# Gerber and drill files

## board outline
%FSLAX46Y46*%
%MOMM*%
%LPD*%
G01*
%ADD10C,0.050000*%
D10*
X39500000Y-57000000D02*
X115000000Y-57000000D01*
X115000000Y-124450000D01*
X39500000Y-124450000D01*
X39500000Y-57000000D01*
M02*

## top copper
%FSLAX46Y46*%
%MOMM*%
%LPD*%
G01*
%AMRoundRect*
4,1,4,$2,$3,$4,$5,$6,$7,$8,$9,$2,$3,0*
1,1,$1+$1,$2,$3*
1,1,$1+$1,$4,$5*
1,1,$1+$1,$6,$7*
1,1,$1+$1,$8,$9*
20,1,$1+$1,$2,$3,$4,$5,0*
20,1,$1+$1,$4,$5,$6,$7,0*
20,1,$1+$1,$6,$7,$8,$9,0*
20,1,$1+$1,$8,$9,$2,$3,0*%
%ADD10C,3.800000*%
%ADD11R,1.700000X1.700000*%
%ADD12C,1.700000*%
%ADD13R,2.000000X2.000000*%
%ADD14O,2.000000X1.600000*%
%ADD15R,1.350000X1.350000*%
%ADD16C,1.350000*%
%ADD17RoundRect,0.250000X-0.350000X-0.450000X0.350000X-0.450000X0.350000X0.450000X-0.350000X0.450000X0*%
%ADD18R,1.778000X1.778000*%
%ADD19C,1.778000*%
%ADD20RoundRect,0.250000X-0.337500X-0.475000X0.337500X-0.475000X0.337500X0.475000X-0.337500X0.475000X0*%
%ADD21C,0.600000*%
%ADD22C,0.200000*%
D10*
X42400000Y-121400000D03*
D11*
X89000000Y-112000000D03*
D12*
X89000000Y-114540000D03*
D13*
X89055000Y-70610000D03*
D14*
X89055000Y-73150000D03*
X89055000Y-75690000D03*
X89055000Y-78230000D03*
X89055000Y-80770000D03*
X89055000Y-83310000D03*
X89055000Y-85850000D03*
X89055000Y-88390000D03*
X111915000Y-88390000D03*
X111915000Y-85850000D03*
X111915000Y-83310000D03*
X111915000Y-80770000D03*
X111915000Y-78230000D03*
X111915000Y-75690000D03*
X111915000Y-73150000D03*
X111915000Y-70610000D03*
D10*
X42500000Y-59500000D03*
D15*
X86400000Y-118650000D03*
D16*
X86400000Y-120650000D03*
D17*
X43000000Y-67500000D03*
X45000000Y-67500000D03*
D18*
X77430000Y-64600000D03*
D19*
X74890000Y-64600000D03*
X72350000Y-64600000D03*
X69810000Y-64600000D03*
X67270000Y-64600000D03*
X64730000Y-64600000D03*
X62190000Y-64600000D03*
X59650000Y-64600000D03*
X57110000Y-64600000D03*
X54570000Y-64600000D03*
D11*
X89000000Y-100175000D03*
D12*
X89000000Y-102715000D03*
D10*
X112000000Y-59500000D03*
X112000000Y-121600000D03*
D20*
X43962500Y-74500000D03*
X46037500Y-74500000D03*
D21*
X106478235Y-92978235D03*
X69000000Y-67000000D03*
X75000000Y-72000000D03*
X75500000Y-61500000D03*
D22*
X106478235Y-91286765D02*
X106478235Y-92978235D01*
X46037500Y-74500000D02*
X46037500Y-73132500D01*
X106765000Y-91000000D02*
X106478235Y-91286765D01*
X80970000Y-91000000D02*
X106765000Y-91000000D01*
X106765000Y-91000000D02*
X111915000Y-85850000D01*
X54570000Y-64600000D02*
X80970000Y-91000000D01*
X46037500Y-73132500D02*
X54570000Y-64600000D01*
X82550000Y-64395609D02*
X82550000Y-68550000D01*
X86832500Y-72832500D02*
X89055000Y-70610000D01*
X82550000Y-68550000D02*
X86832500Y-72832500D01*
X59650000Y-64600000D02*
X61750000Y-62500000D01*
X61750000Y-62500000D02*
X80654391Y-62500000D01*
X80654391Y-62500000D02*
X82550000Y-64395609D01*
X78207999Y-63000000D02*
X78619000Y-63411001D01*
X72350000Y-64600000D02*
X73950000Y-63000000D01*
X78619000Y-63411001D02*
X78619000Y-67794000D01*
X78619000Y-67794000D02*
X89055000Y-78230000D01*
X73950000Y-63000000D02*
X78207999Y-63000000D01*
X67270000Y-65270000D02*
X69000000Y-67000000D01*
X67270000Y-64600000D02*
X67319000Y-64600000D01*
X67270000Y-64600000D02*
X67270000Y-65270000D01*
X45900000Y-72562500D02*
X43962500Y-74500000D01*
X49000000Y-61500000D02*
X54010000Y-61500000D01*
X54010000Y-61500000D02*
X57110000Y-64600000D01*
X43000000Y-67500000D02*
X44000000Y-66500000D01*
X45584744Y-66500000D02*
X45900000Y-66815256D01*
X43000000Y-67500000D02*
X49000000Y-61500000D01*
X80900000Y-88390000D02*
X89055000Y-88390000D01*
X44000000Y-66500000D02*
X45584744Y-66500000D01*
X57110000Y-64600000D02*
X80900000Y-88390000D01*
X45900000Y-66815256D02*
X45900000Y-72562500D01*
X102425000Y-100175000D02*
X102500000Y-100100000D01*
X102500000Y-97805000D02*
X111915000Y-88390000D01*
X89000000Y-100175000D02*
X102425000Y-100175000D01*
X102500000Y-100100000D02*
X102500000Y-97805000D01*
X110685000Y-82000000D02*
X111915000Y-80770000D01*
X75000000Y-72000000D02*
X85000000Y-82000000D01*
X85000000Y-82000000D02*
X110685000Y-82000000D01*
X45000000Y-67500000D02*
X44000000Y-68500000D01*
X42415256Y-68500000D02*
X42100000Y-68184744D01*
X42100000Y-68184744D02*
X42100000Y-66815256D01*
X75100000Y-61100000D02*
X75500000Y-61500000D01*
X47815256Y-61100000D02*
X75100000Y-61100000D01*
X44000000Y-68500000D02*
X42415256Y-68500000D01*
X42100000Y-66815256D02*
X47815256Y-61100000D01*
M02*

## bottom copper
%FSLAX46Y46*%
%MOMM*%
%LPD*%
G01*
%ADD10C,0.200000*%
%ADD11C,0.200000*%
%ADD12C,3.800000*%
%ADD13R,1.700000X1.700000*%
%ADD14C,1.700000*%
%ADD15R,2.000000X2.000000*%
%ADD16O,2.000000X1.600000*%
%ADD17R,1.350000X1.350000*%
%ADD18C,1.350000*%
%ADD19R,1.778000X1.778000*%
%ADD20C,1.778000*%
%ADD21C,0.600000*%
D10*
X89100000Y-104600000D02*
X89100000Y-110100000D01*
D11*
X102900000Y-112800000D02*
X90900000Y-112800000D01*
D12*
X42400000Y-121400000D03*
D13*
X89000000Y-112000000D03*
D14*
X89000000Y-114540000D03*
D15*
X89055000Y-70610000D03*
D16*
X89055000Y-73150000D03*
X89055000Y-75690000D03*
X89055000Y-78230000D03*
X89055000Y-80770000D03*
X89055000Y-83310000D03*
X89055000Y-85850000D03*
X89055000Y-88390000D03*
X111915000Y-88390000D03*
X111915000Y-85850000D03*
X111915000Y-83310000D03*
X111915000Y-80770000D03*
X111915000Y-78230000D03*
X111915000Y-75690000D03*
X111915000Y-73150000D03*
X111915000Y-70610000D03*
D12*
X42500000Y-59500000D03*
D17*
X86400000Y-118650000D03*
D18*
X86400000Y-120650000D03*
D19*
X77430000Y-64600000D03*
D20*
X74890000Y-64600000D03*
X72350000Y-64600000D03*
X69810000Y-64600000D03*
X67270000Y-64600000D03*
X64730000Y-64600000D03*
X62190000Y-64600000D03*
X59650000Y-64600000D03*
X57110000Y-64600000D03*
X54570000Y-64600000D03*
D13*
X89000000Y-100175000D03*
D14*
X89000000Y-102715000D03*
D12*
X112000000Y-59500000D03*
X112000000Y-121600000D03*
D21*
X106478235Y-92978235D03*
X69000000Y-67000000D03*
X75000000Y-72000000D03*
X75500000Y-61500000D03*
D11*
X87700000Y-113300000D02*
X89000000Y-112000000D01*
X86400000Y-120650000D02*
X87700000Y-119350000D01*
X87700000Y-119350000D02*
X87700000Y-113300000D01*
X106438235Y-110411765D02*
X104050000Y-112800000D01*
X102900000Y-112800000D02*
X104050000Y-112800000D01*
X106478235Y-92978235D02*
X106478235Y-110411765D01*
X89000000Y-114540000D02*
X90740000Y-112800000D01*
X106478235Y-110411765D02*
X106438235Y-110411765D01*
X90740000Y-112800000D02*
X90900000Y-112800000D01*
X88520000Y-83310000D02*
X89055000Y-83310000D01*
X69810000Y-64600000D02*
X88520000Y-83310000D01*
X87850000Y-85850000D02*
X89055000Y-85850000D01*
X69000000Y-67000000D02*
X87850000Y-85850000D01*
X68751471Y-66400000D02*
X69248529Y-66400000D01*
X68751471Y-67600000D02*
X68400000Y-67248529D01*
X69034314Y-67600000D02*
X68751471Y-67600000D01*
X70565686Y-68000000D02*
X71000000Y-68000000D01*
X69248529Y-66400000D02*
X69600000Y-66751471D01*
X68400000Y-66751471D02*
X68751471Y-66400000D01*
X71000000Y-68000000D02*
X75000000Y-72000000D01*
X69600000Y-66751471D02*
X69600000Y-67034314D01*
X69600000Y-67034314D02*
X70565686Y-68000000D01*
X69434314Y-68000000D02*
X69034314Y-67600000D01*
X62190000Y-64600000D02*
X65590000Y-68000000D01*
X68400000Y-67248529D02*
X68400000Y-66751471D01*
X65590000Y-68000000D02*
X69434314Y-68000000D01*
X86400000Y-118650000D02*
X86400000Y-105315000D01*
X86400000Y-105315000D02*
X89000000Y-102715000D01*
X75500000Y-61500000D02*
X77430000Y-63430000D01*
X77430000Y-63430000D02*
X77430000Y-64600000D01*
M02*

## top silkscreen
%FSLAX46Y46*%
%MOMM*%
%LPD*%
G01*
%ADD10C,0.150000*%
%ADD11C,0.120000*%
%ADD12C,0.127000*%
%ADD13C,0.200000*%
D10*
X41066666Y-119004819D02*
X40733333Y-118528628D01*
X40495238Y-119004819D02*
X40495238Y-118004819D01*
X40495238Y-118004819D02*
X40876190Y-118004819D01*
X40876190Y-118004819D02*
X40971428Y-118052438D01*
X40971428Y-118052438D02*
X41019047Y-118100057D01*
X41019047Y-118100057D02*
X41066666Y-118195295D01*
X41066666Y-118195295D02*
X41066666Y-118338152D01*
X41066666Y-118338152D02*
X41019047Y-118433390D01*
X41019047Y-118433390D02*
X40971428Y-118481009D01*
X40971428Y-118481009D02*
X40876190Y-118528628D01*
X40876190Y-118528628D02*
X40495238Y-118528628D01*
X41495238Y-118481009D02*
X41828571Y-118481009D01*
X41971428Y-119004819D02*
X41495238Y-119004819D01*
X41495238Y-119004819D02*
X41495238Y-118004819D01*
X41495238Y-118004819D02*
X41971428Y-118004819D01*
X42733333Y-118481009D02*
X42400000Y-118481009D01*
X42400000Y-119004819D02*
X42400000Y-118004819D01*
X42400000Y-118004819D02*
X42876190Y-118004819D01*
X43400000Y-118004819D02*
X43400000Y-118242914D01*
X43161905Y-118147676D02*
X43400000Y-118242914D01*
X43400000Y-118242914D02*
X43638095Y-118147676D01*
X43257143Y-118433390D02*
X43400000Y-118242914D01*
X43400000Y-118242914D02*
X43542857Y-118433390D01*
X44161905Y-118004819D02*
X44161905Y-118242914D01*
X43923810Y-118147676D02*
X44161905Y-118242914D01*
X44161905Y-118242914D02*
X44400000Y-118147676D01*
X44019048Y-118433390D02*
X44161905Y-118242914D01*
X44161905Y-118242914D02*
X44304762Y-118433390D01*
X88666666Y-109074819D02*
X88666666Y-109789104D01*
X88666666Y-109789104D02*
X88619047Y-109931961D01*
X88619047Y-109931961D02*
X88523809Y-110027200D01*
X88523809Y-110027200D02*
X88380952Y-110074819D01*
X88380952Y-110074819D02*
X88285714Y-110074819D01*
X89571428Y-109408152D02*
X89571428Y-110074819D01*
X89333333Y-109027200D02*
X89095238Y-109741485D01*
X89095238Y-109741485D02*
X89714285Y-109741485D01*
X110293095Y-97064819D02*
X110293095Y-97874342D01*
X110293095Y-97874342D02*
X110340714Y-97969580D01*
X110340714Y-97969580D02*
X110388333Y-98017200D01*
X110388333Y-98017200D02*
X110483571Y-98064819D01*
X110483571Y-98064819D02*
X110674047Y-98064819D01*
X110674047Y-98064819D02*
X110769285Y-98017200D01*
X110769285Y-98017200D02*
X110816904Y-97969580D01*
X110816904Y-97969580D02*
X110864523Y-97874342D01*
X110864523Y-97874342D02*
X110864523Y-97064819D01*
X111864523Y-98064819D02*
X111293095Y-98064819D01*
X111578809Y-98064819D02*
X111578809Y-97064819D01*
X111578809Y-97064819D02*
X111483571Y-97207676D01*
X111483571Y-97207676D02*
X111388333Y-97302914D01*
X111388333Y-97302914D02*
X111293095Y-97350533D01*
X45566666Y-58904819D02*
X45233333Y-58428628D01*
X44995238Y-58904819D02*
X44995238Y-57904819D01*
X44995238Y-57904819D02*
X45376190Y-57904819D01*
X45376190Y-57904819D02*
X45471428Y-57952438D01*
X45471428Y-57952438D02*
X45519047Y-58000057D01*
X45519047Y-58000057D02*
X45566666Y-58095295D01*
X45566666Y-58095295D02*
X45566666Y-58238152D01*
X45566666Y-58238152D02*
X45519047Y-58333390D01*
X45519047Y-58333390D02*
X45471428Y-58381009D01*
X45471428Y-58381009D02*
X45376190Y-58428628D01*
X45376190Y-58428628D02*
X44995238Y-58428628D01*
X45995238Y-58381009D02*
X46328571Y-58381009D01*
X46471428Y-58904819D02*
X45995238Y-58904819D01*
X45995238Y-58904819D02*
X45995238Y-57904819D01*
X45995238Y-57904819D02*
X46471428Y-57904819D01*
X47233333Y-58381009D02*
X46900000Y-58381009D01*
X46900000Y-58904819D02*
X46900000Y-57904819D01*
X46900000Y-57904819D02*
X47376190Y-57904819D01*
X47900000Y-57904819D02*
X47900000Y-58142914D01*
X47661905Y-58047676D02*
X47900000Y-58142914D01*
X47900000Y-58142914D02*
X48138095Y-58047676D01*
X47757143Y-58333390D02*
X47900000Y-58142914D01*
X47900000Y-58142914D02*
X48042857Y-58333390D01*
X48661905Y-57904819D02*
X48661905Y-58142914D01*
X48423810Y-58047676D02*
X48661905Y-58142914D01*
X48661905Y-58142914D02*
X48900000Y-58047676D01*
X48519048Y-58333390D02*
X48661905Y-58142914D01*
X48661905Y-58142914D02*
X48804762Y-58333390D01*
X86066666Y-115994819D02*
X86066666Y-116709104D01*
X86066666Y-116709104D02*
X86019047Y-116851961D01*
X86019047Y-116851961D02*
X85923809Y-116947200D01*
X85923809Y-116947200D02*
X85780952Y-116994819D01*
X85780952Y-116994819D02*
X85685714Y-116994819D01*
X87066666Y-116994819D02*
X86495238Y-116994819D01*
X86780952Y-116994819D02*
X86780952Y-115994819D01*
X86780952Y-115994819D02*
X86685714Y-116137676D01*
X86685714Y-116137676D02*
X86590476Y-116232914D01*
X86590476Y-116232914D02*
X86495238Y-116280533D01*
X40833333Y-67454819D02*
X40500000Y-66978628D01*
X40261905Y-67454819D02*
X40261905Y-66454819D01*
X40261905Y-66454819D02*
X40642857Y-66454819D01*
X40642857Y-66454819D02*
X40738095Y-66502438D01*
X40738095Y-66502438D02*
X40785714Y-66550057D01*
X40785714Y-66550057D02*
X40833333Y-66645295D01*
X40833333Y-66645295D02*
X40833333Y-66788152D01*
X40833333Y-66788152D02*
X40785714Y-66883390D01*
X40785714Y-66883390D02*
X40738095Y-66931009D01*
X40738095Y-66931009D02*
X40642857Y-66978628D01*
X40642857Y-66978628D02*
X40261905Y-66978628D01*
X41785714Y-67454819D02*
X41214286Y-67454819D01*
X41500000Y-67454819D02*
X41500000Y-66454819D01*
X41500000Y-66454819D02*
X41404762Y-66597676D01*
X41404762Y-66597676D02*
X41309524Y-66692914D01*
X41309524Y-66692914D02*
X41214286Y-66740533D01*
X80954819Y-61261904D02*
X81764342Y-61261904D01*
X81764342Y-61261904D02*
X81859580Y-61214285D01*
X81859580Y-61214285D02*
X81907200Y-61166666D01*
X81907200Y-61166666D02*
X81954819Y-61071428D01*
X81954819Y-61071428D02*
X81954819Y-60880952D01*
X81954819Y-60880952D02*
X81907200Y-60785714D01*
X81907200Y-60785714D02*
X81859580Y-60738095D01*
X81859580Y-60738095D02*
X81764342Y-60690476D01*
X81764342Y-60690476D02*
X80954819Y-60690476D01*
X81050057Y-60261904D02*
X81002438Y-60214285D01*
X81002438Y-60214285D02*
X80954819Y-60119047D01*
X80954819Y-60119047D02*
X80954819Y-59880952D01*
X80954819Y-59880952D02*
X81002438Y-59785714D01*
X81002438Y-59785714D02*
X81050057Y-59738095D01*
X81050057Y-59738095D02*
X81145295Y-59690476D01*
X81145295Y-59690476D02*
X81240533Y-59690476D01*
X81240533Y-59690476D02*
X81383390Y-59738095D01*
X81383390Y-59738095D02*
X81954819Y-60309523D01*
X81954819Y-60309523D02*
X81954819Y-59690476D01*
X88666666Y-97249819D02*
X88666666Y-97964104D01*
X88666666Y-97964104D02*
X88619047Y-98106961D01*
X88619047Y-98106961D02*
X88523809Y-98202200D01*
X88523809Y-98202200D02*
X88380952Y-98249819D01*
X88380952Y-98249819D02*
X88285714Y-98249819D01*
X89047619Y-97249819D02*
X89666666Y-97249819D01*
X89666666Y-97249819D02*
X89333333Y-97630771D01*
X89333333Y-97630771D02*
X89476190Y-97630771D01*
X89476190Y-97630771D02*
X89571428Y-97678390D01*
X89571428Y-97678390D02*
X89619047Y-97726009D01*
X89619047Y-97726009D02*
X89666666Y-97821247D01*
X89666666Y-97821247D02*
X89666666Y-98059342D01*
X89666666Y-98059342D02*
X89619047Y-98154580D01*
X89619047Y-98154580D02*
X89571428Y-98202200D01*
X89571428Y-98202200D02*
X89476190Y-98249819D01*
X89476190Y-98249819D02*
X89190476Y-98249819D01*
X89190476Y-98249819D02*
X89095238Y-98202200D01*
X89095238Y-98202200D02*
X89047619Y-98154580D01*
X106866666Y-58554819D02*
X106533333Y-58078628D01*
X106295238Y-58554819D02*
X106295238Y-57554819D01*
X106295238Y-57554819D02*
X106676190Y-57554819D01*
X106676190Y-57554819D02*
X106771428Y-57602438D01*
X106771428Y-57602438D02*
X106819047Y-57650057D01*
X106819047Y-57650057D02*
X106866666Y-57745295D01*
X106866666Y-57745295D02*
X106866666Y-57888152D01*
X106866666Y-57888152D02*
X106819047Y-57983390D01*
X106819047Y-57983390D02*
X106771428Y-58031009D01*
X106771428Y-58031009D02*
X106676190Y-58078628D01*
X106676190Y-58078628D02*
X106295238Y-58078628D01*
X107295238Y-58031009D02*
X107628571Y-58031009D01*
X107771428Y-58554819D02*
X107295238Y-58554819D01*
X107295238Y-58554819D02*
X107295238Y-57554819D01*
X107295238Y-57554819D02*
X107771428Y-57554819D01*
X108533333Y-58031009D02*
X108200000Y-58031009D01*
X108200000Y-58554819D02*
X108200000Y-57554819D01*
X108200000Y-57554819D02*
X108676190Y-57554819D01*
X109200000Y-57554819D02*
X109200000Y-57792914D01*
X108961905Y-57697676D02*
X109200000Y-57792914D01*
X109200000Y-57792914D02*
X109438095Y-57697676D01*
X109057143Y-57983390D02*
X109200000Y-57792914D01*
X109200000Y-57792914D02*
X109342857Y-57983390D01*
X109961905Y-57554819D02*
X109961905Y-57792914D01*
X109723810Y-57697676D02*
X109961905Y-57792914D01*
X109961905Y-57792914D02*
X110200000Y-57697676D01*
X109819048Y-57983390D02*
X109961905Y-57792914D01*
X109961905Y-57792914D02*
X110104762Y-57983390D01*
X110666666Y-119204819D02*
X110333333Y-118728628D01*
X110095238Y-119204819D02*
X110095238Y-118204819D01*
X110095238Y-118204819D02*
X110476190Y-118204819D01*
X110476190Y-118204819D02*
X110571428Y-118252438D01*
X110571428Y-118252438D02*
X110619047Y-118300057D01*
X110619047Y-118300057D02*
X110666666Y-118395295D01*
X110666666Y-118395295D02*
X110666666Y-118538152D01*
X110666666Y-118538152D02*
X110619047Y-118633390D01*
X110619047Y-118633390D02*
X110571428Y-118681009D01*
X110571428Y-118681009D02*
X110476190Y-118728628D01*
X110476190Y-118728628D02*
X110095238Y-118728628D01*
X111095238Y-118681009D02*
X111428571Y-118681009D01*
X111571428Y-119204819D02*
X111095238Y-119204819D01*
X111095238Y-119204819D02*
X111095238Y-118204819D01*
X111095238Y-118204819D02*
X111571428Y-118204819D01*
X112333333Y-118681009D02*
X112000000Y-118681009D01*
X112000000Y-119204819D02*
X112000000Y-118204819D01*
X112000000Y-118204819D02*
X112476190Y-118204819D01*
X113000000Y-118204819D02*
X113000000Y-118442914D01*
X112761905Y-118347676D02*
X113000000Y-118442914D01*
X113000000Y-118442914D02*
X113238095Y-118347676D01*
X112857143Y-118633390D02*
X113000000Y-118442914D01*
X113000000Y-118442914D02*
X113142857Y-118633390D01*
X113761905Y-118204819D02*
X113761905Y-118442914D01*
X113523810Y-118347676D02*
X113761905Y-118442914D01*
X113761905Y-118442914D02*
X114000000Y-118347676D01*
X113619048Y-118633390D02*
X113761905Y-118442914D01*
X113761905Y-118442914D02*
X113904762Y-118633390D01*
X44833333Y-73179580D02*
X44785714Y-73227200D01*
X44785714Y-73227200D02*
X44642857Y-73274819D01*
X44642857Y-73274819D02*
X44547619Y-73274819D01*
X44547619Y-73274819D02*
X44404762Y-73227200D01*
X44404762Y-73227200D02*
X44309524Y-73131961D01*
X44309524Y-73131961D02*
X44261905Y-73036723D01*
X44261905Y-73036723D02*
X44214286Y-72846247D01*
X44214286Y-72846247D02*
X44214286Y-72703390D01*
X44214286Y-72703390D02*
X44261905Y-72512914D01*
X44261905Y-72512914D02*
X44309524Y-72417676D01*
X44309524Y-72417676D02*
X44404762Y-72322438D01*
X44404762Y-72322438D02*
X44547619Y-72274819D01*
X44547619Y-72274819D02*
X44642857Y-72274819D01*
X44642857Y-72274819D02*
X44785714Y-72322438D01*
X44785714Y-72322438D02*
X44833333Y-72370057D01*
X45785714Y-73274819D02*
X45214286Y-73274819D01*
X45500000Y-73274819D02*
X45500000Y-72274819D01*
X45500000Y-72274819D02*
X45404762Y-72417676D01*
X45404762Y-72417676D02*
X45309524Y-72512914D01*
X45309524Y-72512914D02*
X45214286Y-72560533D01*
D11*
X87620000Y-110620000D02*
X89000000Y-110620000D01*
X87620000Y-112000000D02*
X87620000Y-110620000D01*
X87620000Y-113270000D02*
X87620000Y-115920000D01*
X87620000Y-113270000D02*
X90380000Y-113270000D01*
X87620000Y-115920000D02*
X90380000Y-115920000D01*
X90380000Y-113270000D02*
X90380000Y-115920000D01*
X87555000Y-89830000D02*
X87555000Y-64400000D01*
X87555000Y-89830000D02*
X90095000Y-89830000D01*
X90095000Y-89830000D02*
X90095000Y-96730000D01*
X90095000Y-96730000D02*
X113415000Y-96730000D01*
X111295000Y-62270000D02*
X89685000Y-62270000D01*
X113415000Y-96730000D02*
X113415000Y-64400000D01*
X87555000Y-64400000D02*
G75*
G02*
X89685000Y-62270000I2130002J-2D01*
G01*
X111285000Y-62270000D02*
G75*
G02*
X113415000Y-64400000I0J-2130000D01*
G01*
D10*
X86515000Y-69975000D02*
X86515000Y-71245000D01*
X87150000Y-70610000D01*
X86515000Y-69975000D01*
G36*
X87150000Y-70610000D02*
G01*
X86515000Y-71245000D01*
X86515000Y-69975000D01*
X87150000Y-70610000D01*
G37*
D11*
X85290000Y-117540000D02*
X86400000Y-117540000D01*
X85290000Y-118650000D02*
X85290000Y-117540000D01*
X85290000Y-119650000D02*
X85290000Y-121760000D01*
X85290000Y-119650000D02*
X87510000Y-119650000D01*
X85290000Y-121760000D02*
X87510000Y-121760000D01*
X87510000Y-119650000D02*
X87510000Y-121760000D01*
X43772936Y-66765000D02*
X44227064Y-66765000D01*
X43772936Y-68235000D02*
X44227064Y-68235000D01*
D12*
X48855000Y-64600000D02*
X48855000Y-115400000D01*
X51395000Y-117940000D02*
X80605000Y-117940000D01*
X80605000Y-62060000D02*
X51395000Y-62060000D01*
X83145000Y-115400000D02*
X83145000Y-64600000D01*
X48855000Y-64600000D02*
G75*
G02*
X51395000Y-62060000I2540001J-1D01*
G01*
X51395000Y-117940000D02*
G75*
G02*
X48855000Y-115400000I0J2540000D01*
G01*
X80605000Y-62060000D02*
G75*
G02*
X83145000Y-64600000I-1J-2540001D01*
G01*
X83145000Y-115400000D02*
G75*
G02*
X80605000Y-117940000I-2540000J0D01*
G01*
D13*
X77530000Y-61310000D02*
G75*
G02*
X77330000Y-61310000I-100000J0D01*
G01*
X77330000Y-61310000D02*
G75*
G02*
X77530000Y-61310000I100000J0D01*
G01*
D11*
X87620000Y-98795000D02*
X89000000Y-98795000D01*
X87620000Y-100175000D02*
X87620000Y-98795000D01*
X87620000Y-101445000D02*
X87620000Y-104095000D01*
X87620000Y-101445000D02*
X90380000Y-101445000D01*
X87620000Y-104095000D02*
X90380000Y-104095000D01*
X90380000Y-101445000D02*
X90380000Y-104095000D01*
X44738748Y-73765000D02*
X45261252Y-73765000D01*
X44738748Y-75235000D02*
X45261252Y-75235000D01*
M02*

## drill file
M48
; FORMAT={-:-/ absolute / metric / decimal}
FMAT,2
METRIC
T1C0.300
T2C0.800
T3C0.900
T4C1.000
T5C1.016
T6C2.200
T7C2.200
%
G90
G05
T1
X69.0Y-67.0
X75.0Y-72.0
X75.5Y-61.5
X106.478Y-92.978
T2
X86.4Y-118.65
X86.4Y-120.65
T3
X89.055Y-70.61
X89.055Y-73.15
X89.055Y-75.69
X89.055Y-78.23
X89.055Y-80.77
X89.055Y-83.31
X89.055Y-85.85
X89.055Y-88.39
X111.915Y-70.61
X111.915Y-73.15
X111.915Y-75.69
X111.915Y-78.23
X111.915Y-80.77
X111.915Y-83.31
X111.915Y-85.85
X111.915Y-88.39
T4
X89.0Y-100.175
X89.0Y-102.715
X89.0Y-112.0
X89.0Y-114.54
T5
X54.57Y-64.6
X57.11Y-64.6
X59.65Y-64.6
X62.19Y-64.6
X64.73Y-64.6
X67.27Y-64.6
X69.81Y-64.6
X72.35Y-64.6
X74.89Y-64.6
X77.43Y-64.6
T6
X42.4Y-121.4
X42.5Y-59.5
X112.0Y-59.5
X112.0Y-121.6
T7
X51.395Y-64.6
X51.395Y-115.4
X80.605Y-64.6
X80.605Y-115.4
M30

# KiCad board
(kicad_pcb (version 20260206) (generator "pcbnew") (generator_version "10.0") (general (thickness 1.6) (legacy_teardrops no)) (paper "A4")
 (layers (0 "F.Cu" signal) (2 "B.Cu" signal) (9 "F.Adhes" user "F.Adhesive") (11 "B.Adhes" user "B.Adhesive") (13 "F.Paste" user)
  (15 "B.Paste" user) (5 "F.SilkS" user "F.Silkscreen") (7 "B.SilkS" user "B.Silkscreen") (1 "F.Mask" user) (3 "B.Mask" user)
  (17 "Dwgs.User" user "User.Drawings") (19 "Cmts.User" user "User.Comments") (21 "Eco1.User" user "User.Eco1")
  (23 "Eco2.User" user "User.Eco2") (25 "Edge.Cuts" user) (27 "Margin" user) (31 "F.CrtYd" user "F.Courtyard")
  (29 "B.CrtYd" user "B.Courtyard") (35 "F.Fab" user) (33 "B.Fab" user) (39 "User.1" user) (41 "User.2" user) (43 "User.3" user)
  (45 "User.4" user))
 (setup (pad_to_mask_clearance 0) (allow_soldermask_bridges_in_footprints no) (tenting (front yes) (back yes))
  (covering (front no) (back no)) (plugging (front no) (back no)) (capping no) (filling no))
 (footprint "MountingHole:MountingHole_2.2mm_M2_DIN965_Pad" (layer "F.Cu") (at 42.4 121.4)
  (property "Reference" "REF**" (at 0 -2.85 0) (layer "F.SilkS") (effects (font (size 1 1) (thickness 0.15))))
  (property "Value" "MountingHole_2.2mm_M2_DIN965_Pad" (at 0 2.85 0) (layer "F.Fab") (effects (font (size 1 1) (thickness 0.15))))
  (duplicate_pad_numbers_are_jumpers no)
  (pad "1" thru_hole circle (at 0 0) (size 3.8 3.8) (drill 2.2) (layers "*.Cu" "*.Mask") (remove_unused_layers no) (zone_connect 2)))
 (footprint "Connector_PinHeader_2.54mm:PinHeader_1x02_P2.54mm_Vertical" (layer "F.Cu") (at 89 112)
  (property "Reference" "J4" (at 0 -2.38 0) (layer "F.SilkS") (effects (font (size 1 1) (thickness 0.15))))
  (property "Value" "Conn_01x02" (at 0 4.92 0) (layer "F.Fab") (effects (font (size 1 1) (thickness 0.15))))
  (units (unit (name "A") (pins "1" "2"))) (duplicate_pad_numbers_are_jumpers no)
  (fp_line (start -1.38 -1.38) (end 0 -1.38) (stroke (width 0.12) (type solid)) (layer "F.SilkS"))
  (fp_line (start -1.38 0) (end -1.38 -1.38) (stroke (width 0.12) (type solid)) (layer "F.SilkS"))
  (fp_line (start -1.38 1.27) (end -1.38 3.92) (stroke (width 0.12) (type solid)) (layer "F.SilkS"))
  (fp_line (start -1.38 1.27) (end 1.38 1.27) (stroke (width 0.12) (type solid)) (layer "F.SilkS"))
  (fp_line (start -1.38 3.92) (end 1.38 3.92) (stroke (width 0.12) (type solid)) (layer "F.SilkS"))
  (fp_line (start 1.38 1.27) (end 1.38 3.92) (stroke (width 0.12) (type solid)) (layer "F.SilkS"))
  (pad "1" thru_hole rect (at 0 0) (size 1.7 1.7) (drill 1) (layers "*.Cu" "*.Mask") (remove_unused_layers no) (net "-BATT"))
  (pad "2" thru_hole circle (at 0 2.54) (size 1.7 1.7) (drill 1) (layers "*.Cu" "*.Mask") (remove_unused_layers no) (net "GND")))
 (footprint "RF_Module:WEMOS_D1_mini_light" (layer "F.Cu") (at 89.055 70.61)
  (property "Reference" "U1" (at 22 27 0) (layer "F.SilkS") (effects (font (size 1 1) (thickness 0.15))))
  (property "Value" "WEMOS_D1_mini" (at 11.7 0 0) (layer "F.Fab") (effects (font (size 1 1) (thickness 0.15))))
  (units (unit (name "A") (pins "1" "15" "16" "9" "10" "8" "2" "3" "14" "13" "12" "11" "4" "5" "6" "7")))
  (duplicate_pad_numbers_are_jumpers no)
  (fp_line (start -1.5 19.22) (end -1.5 -6.21) (stroke (width 0.12) (type solid)) (layer "F.SilkS"))
  (fp_line (start -1.5 19.22) (end 1.04 19.22) (stroke (width 0.12) (type solid)) (layer "F.SilkS"))
  (fp_line (start 1.04 19.22) (end 1.04 26.12) (stroke (width 0.12) (type solid)) (layer "F.SilkS"))
  (fp_line (start 1.04 26.12) (end 24.36 26.12) (stroke (width 0.12) (type solid)) (layer "F.SilkS"))
  (fp_line (start 22.24 -8.34) (end 0.63 -8.34) (stroke (width 0.12) (type solid)) (layer "F.SilkS"))
  (fp_line (start 24.36 26.12) (end 24.36 -6.21) (stroke (width 0.12) (type solid)) (layer "F.SilkS"))
  (fp_arc (start -1.5 -6.21) (mid -0.876137 -7.716137) (end 0.63 -8.34) (stroke (width 0.12) (type solid)) (layer "F.SilkS"))
  (fp_arc (start 22.23 -8.34) (mid 23.736137 -7.716137) (end 24.36 -6.21) (stroke (width 0.12) (type solid)) (layer "F.SilkS"))
  (fp_poly (pts (xy -2.54 -0.635) (xy -2.54 0.635) (xy -1.905 0)) (stroke (width 0.15) (type solid)) (fill yes) (layer "F.SilkS"))
  (pad "1" thru_hole rect (at 0 0) (size 2 2) (drill 0.9) (layers "*.Cu" "*.Mask") (remove_unused_layers no) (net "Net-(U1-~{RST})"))
  (pad "2" thru_hole oval (at 0 2.54) (size 2 1.6) (drill 0.9) (layers "*.Cu" "*.Mask") (remove_unused_layers no)
   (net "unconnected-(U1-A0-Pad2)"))
  (pad "3" thru_hole oval (at 0 5.08) (size 2 1.6) (drill 0.9) (layers "*.Cu" "*.Mask") (remove_unused_layers no)
   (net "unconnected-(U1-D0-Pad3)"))
  (pad "4" thru_hole oval (at 0 7.62) (size 2 1.6) (drill 0.9) (layers "*.Cu" "*.Mask") (remove_unused_layers no)
   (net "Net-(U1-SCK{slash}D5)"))
  (pad "5" thru_hole oval (at 0 10.16) (size 2 1.6) (drill 0.9) (layers "*.Cu" "*.Mask") (remove_unused_layers no)
   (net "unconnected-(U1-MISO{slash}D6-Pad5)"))
  (pad "6" thru_hole oval (at 0 12.7) (size 2 1.6) (drill 0.9) (layers "*.Cu" "*.Mask") (remove_unused_layers no)
   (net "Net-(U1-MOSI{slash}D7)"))
  (pad "7" thru_hole oval (at 0 15.24) (size 2 1.6) (drill 0.9) (layers "*.Cu" "*.Mask") (remove_unused_layers no)
   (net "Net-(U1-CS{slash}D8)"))
  (pad "8" thru_hole oval (at 0 17.78) (size 2 1.6) (drill 0.9) (layers "*.Cu" "*.Mask") (remove_unused_layers no) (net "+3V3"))
  (pad "9" thru_hole oval (at 22.86 17.78) (size 2 1.6) (drill 0.9) (layers "*.Cu" "*.Mask") (remove_unused_layers no) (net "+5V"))
  (pad "10" thru_hole oval (at 22.86 15.24) (size 2 1.6) (drill 0.9) (layers "*.Cu" "*.Mask") (remove_unused_layers no) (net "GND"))
  (pad "11" thru_hole oval (at 22.86 12.7) (size 2 1.6) (drill 0.9) (layers "*.Cu" "*.Mask") (remove_unused_layers no)
   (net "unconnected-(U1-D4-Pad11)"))
  (pad "12" thru_hole oval (at 22.86 10.16) (size 2 1.6) (drill 0.9) (layers "*.Cu" "*.Mask") (remove_unused_layers no) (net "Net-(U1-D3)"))
  (pad "13" thru_hole oval (at 22.86 7.62) (size 2 1.6) (drill 0.9) (layers "*.Cu" "*.Mask") (remove_unused_layers no)
   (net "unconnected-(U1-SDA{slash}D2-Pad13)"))
  (pad "14" thru_hole oval (at 22.86 5.08) (size 2 1.6) (drill 0.9) (layers "*.Cu" "*.Mask") (remove_unused_layers no)
   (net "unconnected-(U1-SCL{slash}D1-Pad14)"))
  (pad "15" thru_hole oval (at 22.86 2.54) (size 2 1.6) (drill 0.9) (layers "*.Cu" "*.Mask") (remove_unused_layers no)
   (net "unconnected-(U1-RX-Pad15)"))
  (pad "16" thru_hole oval (at 22.86 0) (size 2 1.6) (drill 0.9) (layers "*.Cu" "*.Mask") (remove_unused_layers no)
   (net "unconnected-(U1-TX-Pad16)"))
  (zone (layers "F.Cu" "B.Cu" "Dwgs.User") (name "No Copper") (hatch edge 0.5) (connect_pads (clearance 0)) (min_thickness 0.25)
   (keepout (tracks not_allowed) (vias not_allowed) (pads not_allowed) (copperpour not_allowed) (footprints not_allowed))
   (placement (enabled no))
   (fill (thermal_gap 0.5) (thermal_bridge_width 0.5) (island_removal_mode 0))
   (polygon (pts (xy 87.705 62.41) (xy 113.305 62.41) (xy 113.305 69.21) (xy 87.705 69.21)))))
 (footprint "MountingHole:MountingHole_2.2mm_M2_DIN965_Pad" (layer "F.Cu") (at 42.5 59.5)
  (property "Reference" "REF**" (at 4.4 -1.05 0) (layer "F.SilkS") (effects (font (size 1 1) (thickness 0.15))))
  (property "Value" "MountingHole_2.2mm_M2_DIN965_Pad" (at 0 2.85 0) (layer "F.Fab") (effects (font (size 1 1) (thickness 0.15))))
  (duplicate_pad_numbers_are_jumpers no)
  (pad "1" thru_hole circle (at 0 0) (size 3.8 3.8) (drill 2.2) (layers "*.Cu" "*.Mask") (remove_unused_layers no) (zone_connect 2)))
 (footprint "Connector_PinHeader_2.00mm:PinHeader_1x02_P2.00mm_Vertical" (layer "F.Cu") (at 86.4 118.65)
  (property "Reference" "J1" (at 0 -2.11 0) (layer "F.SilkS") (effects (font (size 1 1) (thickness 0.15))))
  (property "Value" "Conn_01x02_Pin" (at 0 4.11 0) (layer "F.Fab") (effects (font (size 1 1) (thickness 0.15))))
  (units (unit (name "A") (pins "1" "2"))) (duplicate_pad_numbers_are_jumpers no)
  (fp_line (start -1.11 -1.11) (end 0 -1.11) (stroke (width 0.12) (type solid)) (layer "F.SilkS"))
  (fp_line (start -1.11 0) (end -1.11 -1.11) (stroke (width 0.12) (type solid)) (layer "F.SilkS"))
  (fp_line (start -1.11 1) (end -1.11 3.11) (stroke (width 0.12) (type solid)) (layer "F.SilkS"))
  (fp_line (start -1.11 1) (end 1.11 1) (stroke (width 0.12) (type solid)) (layer "F.SilkS"))
  (fp_line (start -1.11 3.11) (end 1.11 3.11) (stroke (width 0.12) (type solid)) (layer "F.SilkS"))
  (fp_line (start 1.11 1) (end 1.11 3.11) (stroke (width 0.12) (type solid)) (layer "F.SilkS"))
  (pad "1" thru_hole rect (at 0 0) (size 1.35 1.35) (drill 0.8) (layers "*.Cu" "*.Mask") (remove_unused_layers no) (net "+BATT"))
  (pad "2" thru_hole circle (at 0 2) (size 1.35 1.35) (drill 0.8) (layers "*.Cu" "*.Mask") (remove_unused_layers no) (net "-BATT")))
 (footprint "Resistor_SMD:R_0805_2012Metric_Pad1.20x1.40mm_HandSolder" (layer "F.Cu") (at 44 67.5)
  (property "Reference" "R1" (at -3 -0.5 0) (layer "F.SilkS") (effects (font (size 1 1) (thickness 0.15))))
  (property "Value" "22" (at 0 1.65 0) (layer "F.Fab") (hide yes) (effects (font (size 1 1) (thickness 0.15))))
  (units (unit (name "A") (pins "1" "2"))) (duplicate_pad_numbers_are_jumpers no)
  (fp_line (start -0.227064 -0.735) (end 0.227064 -0.735) (stroke (width 0.12) (type solid)) (layer "F.SilkS"))
  (fp_line (start -0.227064 0.735) (end 0.227064 0.735) (stroke (width 0.12) (type solid)) (layer "F.SilkS"))
  (pad "1" smd roundrect (at -1 0) (size 1.2 1.4) (layers "F.Cu" "F.Mask" "F.Paste") (roundrect_rratio 0.208333) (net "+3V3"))
  (pad "2" smd roundrect (at 1 0) (size 1.2 1.4) (layers "F.Cu" "F.Mask" "F.Paste") (roundrect_rratio 0.208333) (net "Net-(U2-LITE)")))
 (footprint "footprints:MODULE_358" (layer "F.Cu") (at 66 90 -90)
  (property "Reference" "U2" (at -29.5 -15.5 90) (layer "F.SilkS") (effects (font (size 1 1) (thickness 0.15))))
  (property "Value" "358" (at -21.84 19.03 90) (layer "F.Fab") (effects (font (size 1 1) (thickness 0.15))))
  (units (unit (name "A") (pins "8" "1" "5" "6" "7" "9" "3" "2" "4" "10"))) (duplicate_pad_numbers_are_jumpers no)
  (fp_line (start -25.4 17.145) (end 25.4 17.145) (stroke (width 0.127) (type solid)) (layer "F.SilkS"))
  (fp_line (start 27.94 14.605) (end 27.94 -14.605) (stroke (width 0.127) (type solid)) (layer "F.SilkS"))
  (fp_line (start -27.94 -14.605) (end -27.94 14.605) (stroke (width 0.127) (type solid)) (layer "F.SilkS"))
  (fp_line (start 25.4 -17.145) (end -25.4 -17.145) (stroke (width 0.127) (type solid)) (layer "F.SilkS"))
  (fp_arc (start -25.4 17.145) (mid -27.196051 16.401051) (end -27.94 14.605) (stroke (width 0.127) (type solid)) (layer "F.SilkS"))
  (fp_arc (start 27.94 14.605) (mid 27.196051 16.401051) (end 25.4 17.145) (stroke (width 0.127) (type solid)) (layer "F.SilkS"))
  (fp_arc (start -27.94 -14.605) (mid -27.196051 -16.401051) (end -25.4 -17.145) (stroke (width 0.127) (type solid)) (layer "F.SilkS"))
  (fp_arc (start 25.4 -17.145) (mid 27.196051 -16.401051) (end 27.94 -14.605) (stroke (width 0.127) (type solid)) (layer "F.SilkS"))
  (fp_circle (center -28.69 -11.43) (end -28.59 -11.43) (stroke (width 0.2) (type solid)) (fill no) (layer "F.SilkS"))
  (pad "" np_thru_hole circle (at -25.4 -14.605 270) (size 2.2 2.2) (drill 2.2) (layers "*.Cu" "*.Mask"))
  (pad "" np_thru_hole circle (at -25.4 14.605 270) (size 2.2 2.2) (drill 2.2) (layers "*.Cu" "*.Mask"))
  (pad "" np_thru_hole circle (at 25.4 -14.605 270) (size 2.2 2.2) (drill 2.2) (layers "*.Cu" "*.Mask"))
  (pad "" np_thru_hole circle (at 25.4 14.605 270) (size 2.2 2.2) (drill 2.2) (layers "*.Cu" "*.Mask"))
  (pad "1" thru_hole rect (at -25.4 -11.43 270) (size 1.778 1.778) (drill 1.016) (layers "*.Cu" "*.Mask") (remove_unused_layers no)
   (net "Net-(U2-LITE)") (solder_mask_margin 0.102))
  (pad "2" thru_hole circle (at -25.4 -8.89 270) (size 1.778 1.778) (drill 1.016) (layers "*.Cu" "*.Mask") (remove_unused_layers no)
   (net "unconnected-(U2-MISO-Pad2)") (solder_mask_margin 0.102))
  (pad "3" thru_hole circle (at -25.4 -6.35 270) (size 1.778 1.778) (drill 1.016) (layers "*.Cu" "*.Mask") (remove_unused_layers no)
   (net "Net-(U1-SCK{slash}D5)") (solder_mask_margin 0.102))
  (pad "4" thru_hole circle (at -25.4 -3.81 270) (size 1.778 1.778) (drill 1.016) (layers "*.Cu" "*.Mask") (remove_unused_layers no)
   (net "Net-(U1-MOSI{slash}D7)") (solder_mask_margin 0.102))
  (pad "5" thru_hole circle (at -25.4 -1.27 270) (size 1.778 1.778) (drill 1.016) (layers "*.Cu" "*.Mask") (remove_unused_layers no)
   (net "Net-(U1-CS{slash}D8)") (solder_mask_margin 0.102))
  (pad "6" thru_hole circle (at -25.4 1.27 270) (size 1.778 1.778) (drill 1.016) (layers "*.Cu" "*.Mask") (remove_unused_layers no)
   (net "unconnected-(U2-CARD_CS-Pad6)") (solder_mask_margin 0.102))
  (pad "7" thru_hole circle (at -25.4 3.81 270) (size 1.778 1.778) (drill 1.016) (layers "*.Cu" "*.Mask") (remove_unused_layers no)
   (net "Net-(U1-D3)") (solder_mask_margin 0.102))
  (pad "8" thru_hole circle (at -25.4 6.35 270) (size 1.778 1.778) (drill 1.016) (layers "*.Cu" "*.Mask") (remove_unused_layers no)
   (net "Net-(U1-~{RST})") (solder_mask_margin 0.102))
  (pad "9" thru_hole circle (at -25.4 8.89 270) (size 1.778 1.778) (drill 1.016) (layers "*.Cu" "*.Mask") (remove_unused_layers no)
   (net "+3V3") (solder_mask_margin 0.102))
  (pad "10" thru_hole circle (at -25.4 11.43 270) (size 1.778 1.778) (drill 1.016) (layers "*.Cu" "*.Mask") (remove_unused_layers no)
   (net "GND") (solder_mask_margin 0.102)))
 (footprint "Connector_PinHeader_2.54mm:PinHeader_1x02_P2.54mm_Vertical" (layer "F.Cu") (at 89 100.175)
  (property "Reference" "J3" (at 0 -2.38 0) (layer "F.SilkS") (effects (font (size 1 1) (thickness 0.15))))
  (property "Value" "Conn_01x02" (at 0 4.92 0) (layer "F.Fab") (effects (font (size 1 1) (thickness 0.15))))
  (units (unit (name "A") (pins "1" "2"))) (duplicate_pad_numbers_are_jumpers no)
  (fp_line (start -1.38 -1.38) (end 0 -1.38) (stroke (width 0.12) (type solid)) (layer "F.SilkS"))
  (fp_line (start -1.38 0) (end -1.38 -1.38) (stroke (width 0.12) (type solid)) (layer "F.SilkS"))
  (fp_line (start -1.38 1.27) (end -1.38 3.92) (stroke (width 0.12) (type solid)) (layer "F.SilkS"))
  (fp_line (start -1.38 1.27) (end 1.38 1.27) (stroke (width 0.12) (type solid)) (layer "F.SilkS"))
  (fp_line (start -1.38 3.92) (end 1.38 3.92) (stroke (width 0.12) (type solid)) (layer "F.SilkS"))
  (fp_line (start 1.38 1.27) (end 1.38 3.92) (stroke (width 0.12) (type solid)) (layer "F.SilkS"))
  (pad "1" thru_hole rect (at 0 0) (size 1.7 1.7) (drill 1) (layers "*.Cu" "*.Mask") (remove_unused_layers no) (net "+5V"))
  (pad "2" thru_hole circle (at 0 2.54) (size 1.7 1.7) (drill 1) (layers "*.Cu" "*.Mask") (remove_unused_layers no) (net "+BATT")))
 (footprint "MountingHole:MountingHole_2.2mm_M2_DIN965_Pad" (layer "F.Cu") (at 112 59.5)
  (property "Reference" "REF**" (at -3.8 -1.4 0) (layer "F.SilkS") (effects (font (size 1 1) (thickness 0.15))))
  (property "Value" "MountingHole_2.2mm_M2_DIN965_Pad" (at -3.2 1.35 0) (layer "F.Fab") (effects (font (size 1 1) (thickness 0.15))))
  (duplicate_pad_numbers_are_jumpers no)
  (pad "1" thru_hole circle (at 0 0) (size 3.8 3.8) (drill 2.2) (layers "*.Cu" "*.Mask") (remove_unused_layers no) (zone_connect 2)))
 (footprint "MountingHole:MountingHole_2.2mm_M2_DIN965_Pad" (layer "F.Cu") (at 112 121.6)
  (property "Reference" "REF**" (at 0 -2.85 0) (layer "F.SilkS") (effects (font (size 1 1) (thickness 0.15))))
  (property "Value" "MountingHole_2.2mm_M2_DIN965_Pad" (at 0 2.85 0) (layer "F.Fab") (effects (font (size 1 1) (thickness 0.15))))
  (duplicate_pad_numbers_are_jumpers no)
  (pad "1" thru_hole circle (at 0 0) (size 3.8 3.8) (drill 2.2) (layers "*.Cu" "*.Mask") (remove_unused_layers no) (zone_connect 2)))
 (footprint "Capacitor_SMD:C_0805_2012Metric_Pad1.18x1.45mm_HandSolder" (layer "F.Cu") (at 45 74.5)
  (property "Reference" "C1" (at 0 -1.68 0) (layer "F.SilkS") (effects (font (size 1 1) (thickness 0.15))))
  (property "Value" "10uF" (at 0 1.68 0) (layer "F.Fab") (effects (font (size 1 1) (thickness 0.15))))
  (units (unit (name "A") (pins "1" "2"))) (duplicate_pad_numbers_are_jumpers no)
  (fp_line (start -0.261252 -0.735) (end 0.261252 -0.735) (stroke (width 0.12) (type solid)) (layer "F.SilkS"))
  (fp_line (start -0.261252 0.735) (end 0.261252 0.735) (stroke (width 0.12) (type solid)) (layer "F.SilkS"))
  (pad "1" smd roundrect (at -1.0375 0) (size 1.175 1.45) (layers "F.Cu" "F.Mask" "F.Paste") (roundrect_rratio 0.212766) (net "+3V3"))
  (pad "2" smd roundrect (at 1.0375 0) (size 1.175 1.45) (layers "F.Cu" "F.Mask" "F.Paste") (roundrect_rratio 0.212766) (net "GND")))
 (gr_line (start 89.1 104.6) (end 89.1 110.1) (stroke (width 0.2) (type default)) (layer "B.Cu"))
 (gr_line (start 102.9 112.8) (end 90.9 112.8) (stroke (width 0.2) (type default)) (layer "B.Cu") (net "GND"))
 (gr_rect (start 39.5 57) (end 115 124.45) (stroke (width 0.05) (type default)) (fill no) (layer "Edge.Cuts"))
 (segment (start 87.7 113.3) (end 89 112) (width 0.2) (layer "B.Cu") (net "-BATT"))
 (segment (start 86.4 120.65) (end 87.7 119.35) (width 0.2) (layer "B.Cu") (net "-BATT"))
 (segment (start 87.7 119.35) (end 87.7 113.3) (width 0.2) (layer "B.Cu") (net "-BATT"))
 (segment (start 106.478235 91.286765) (end 106.478235 92.978235) (width 0.2) (layer "F.Cu") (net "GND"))
 (segment (start 46.0375 74.5) (end 46.0375 73.1325) (width 0.2) (layer "F.Cu") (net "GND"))
 (segment (start 106.765 91) (end 106.478235 91.286765) (width 0.2) (layer "F.Cu") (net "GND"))
 (segment (start 80.97 91) (end 106.765 91) (width 0.2) (layer "F.Cu") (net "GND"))
 (segment (start 106.765 91) (end 111.915 85.85) (width 0.2) (layer "F.Cu") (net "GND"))
 (segment (start 54.57 64.6) (end 80.97 91) (width 0.2) (layer "F.Cu") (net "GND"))
 (segment (start 46.0375 73.1325) (end 54.57 64.6) (width 0.2) (layer "F.Cu") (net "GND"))
 (via (at 106.478235 92.978235) (size 0.6) (drill 0.3) (layers "F.Cu" "B.Cu") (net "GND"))
 (segment (start 106.438235 110.411765) (end 104.05 112.8) (width 0.2) (layer "B.Cu") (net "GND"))
 (segment (start 102.9 112.8) (end 104.05 112.8) (width 0.2) (layer "B.Cu") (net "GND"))
 (segment (start 106.478235 92.978235) (end 106.478235 110.411765) (width 0.2) (layer "B.Cu") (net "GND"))
 (segment (start 89 114.54) (end 90.74 112.8) (width 0.2) (layer "B.Cu") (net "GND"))
 (segment (start 106.478235 110.411765) (end 106.438235 110.411765) (width 0.2) (layer "B.Cu") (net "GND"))
 (segment (start 90.74 112.8) (end 90.9 112.8) (width 0.2) (layer "B.Cu") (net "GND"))
 (segment (start 82.55 64.395609) (end 82.55 68.55) (width 0.2) (layer "F.Cu") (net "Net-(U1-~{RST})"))
 (segment (start 86.8325 72.8325) (end 89.055 70.61) (width 0.2) (layer "F.Cu") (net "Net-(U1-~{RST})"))
 (segment (start 82.55 68.55) (end 86.8325 72.8325) (width 0.2) (layer "F.Cu") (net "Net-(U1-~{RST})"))
 (segment (start 59.65 64.6) (end 61.75 62.5) (width 0.2) (layer "F.Cu") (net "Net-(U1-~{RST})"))
 (segment (start 61.75 62.5) (end 80.654391 62.5) (width 0.2) (layer "F.Cu") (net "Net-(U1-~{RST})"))
 (segment (start 80.654391 62.5) (end 82.55 64.395609) (width 0.2) (layer "F.Cu") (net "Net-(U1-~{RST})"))
 (segment (start 78.207999 63) (end 78.619 63.411001) (width 0.2) (layer "F.Cu") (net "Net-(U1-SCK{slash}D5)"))
 (segment (start 72.35 64.6) (end 73.95 63) (width 0.2) (layer "F.Cu") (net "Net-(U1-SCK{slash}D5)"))
 (segment (start 78.619 63.411001) (end 78.619 67.794) (width 0.2) (layer "F.Cu") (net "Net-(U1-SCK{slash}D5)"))
 (segment (start 78.619 67.794) (end 89.055 78.23) (width 0.2) (layer "F.Cu") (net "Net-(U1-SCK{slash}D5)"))
 (segment (start 73.95 63) (end 78.207999 63) (width 0.2) (layer "F.Cu") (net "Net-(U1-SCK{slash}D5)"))
 (segment (start 88.52 83.31) (end 89.055 83.31) (width 0.2) (layer "B.Cu") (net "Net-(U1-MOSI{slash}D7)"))
 (segment (start 69.81 64.6) (end 88.52 83.31) (width 0.2) (layer "B.Cu") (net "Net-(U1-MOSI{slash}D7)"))
 (segment (start 67.27 65.27) (end 69 67) (width 0.2) (layer "F.Cu") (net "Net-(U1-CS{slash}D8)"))
 (segment (start 67.27 64.6) (end 67.319 64.6) (width 0.2) (layer "F.Cu") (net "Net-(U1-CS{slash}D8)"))
 (segment (start 67.27 64.6) (end 67.27 65.27) (width 0.2) (layer "F.Cu") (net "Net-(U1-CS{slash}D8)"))
 (via (at 69 67) (size 0.6) (drill 0.3) (layers "F.Cu" "B.Cu") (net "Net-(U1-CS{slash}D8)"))
 (segment (start 87.85 85.85) (end 89.055 85.85) (width 0.2) (layer "B.Cu") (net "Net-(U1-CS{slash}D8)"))
 (segment (start 69 67) (end 87.85 85.85) (width 0.2) (layer "B.Cu") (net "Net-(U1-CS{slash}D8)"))
 (segment (start 45.9 72.5625) (end 43.9625 74.5) (width 0.2) (layer "F.Cu") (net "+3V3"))
 (segment (start 49 61.5) (end 54.01 61.5) (width 0.2) (layer "F.Cu") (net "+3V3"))
 (segment (start 54.01 61.5) (end 57.11 64.6) (width 0.2) (layer "F.Cu") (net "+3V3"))
 (segment (start 43 67.5) (end 44 66.5) (width 0.2) (layer "F.Cu") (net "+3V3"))
 (segment (start 45.584744 66.5) (end 45.9 66.815256) (width 0.2) (layer "F.Cu") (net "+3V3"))
 (segment (start 43 67.5) (end 49 61.5) (width 0.2) (layer "F.Cu") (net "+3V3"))
 (segment (start 80.9 88.39) (end 89.055 88.39) (width 0.2) (layer "F.Cu") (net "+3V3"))
 (segment (start 44 66.5) (end 45.584744 66.5) (width 0.2) (layer "F.Cu") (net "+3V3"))
 (segment (start 57.11 64.6) (end 80.9 88.39) (width 0.2) (layer "F.Cu") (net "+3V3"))
 (segment (start 45.9 66.815256) (end 45.9 72.5625) (width 0.2) (layer "F.Cu") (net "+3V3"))
 (segment (start 102.425 100.175) (end 102.5 100.1) (width 0.2) (layer "F.Cu") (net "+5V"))
 (segment (start 102.5 97.805) (end 111.915 88.39) (width 0.2) (layer "F.Cu") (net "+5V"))
 (segment (start 89 100.175) (end 102.425 100.175) (width 0.2) (layer "F.Cu") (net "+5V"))
 (segment (start 102.5 100.1) (end 102.5 97.805) (width 0.2) (layer "F.Cu") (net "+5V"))
 (segment (start 110.685 82) (end 111.915 80.77) (width 0.2) (layer "F.Cu") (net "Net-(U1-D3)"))
 (segment (start 75 72) (end 85 82) (width 0.2) (layer "F.Cu") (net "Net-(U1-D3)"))
 (segment (start 85 82) (end 110.685 82) (width 0.2) (layer "F.Cu") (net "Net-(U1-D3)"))
 (via (at 75 72) (size 0.6) (drill 0.3) (layers "F.Cu" "B.Cu") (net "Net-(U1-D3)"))
 (segment (start 68.751471 66.4) (end 69.248529 66.4) (width 0.2) (layer "B.Cu") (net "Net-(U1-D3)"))
 (segment (start 68.751471 67.6) (end 68.4 67.248529) (width 0.2) (layer "B.Cu") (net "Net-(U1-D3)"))
 (segment (start 69.034314 67.6) (end 68.751471 67.6) (width 0.2) (layer "B.Cu") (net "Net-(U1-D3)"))
 (segment (start 70.565686 68) (end 71 68) (width 0.2) (layer "B.Cu") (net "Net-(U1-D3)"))
 (segment (start 69.248529 66.4) (end 69.6 66.751471) (width 0.2) (layer "B.Cu") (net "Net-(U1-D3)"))
 (segment (start 68.4 66.751471) (end 68.751471 66.4) (width 0.2) (layer "B.Cu") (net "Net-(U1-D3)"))
 (segment (start 71 68) (end 75 72) (width 0.2) (layer "B.Cu") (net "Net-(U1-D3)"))
 (segment (start 69.6 66.751471) (end 69.6 67.034314) (width 0.2) (layer "B.Cu") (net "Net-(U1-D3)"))
 (segment (start 69.6 67.034314) (end 70.565686 68) (width 0.2) (layer "B.Cu") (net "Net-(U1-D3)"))
 (segment (start 69.434314 68) (end 69.034314 67.6) (width 0.2) (layer "B.Cu") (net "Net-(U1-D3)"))
 (segment (start 62.19 64.6) (end 65.59 68) (width 0.2) (layer "B.Cu") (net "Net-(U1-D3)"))
 (segment (start 68.4 67.248529) (end 68.4 66.751471) (width 0.2) (layer "B.Cu") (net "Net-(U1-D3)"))
 (segment (start 65.59 68) (end 69.434314 68) (width 0.2) (layer "B.Cu") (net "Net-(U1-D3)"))
 (segment (start 86.4 118.65) (end 86.4 105.315) (width 0.2) (layer "B.Cu") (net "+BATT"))
 (segment (start 86.4 105.315) (end 89 102.715) (width 0.2) (layer "B.Cu") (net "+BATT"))
 (segment (start 45 67.5) (end 44 68.5) (width 0.2) (layer "F.Cu") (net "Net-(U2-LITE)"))
 (segment (start 42.415256 68.5) (end 42.1 68.184744) (width 0.2) (layer "F.Cu") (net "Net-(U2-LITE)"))
 (segment (start 42.1 68.184744) (end 42.1 66.815256) (width 0.2) (layer "F.Cu") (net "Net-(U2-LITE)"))
 (segment (start 75.1 61.1) (end 75.5 61.5) (width 0.2) (layer "F.Cu") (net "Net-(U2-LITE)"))
 (segment (start 47.815256 61.1) (end 75.1 61.1) (width 0.2) (layer "F.Cu") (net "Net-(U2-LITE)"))
 (segment (start 44 68.5) (end 42.415256 68.5) (width 0.2) (layer "F.Cu") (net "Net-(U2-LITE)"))
 (segment (start 42.1 66.815256) (end 47.815256 61.1) (width 0.2) (layer "F.Cu") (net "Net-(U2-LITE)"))
 (via (at 75.5 61.5) (size 0.6) (drill 0.3) (layers "F.Cu" "B.Cu") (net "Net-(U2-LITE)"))
 (segment (start 75.5 61.5) (end 77.43 63.43) (width 0.2) (layer "B.Cu") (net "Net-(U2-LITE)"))
 (segment (start 77.43 63.43) (end 77.43 64.6) (width 0.2) (layer "B.Cu") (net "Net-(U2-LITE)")))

